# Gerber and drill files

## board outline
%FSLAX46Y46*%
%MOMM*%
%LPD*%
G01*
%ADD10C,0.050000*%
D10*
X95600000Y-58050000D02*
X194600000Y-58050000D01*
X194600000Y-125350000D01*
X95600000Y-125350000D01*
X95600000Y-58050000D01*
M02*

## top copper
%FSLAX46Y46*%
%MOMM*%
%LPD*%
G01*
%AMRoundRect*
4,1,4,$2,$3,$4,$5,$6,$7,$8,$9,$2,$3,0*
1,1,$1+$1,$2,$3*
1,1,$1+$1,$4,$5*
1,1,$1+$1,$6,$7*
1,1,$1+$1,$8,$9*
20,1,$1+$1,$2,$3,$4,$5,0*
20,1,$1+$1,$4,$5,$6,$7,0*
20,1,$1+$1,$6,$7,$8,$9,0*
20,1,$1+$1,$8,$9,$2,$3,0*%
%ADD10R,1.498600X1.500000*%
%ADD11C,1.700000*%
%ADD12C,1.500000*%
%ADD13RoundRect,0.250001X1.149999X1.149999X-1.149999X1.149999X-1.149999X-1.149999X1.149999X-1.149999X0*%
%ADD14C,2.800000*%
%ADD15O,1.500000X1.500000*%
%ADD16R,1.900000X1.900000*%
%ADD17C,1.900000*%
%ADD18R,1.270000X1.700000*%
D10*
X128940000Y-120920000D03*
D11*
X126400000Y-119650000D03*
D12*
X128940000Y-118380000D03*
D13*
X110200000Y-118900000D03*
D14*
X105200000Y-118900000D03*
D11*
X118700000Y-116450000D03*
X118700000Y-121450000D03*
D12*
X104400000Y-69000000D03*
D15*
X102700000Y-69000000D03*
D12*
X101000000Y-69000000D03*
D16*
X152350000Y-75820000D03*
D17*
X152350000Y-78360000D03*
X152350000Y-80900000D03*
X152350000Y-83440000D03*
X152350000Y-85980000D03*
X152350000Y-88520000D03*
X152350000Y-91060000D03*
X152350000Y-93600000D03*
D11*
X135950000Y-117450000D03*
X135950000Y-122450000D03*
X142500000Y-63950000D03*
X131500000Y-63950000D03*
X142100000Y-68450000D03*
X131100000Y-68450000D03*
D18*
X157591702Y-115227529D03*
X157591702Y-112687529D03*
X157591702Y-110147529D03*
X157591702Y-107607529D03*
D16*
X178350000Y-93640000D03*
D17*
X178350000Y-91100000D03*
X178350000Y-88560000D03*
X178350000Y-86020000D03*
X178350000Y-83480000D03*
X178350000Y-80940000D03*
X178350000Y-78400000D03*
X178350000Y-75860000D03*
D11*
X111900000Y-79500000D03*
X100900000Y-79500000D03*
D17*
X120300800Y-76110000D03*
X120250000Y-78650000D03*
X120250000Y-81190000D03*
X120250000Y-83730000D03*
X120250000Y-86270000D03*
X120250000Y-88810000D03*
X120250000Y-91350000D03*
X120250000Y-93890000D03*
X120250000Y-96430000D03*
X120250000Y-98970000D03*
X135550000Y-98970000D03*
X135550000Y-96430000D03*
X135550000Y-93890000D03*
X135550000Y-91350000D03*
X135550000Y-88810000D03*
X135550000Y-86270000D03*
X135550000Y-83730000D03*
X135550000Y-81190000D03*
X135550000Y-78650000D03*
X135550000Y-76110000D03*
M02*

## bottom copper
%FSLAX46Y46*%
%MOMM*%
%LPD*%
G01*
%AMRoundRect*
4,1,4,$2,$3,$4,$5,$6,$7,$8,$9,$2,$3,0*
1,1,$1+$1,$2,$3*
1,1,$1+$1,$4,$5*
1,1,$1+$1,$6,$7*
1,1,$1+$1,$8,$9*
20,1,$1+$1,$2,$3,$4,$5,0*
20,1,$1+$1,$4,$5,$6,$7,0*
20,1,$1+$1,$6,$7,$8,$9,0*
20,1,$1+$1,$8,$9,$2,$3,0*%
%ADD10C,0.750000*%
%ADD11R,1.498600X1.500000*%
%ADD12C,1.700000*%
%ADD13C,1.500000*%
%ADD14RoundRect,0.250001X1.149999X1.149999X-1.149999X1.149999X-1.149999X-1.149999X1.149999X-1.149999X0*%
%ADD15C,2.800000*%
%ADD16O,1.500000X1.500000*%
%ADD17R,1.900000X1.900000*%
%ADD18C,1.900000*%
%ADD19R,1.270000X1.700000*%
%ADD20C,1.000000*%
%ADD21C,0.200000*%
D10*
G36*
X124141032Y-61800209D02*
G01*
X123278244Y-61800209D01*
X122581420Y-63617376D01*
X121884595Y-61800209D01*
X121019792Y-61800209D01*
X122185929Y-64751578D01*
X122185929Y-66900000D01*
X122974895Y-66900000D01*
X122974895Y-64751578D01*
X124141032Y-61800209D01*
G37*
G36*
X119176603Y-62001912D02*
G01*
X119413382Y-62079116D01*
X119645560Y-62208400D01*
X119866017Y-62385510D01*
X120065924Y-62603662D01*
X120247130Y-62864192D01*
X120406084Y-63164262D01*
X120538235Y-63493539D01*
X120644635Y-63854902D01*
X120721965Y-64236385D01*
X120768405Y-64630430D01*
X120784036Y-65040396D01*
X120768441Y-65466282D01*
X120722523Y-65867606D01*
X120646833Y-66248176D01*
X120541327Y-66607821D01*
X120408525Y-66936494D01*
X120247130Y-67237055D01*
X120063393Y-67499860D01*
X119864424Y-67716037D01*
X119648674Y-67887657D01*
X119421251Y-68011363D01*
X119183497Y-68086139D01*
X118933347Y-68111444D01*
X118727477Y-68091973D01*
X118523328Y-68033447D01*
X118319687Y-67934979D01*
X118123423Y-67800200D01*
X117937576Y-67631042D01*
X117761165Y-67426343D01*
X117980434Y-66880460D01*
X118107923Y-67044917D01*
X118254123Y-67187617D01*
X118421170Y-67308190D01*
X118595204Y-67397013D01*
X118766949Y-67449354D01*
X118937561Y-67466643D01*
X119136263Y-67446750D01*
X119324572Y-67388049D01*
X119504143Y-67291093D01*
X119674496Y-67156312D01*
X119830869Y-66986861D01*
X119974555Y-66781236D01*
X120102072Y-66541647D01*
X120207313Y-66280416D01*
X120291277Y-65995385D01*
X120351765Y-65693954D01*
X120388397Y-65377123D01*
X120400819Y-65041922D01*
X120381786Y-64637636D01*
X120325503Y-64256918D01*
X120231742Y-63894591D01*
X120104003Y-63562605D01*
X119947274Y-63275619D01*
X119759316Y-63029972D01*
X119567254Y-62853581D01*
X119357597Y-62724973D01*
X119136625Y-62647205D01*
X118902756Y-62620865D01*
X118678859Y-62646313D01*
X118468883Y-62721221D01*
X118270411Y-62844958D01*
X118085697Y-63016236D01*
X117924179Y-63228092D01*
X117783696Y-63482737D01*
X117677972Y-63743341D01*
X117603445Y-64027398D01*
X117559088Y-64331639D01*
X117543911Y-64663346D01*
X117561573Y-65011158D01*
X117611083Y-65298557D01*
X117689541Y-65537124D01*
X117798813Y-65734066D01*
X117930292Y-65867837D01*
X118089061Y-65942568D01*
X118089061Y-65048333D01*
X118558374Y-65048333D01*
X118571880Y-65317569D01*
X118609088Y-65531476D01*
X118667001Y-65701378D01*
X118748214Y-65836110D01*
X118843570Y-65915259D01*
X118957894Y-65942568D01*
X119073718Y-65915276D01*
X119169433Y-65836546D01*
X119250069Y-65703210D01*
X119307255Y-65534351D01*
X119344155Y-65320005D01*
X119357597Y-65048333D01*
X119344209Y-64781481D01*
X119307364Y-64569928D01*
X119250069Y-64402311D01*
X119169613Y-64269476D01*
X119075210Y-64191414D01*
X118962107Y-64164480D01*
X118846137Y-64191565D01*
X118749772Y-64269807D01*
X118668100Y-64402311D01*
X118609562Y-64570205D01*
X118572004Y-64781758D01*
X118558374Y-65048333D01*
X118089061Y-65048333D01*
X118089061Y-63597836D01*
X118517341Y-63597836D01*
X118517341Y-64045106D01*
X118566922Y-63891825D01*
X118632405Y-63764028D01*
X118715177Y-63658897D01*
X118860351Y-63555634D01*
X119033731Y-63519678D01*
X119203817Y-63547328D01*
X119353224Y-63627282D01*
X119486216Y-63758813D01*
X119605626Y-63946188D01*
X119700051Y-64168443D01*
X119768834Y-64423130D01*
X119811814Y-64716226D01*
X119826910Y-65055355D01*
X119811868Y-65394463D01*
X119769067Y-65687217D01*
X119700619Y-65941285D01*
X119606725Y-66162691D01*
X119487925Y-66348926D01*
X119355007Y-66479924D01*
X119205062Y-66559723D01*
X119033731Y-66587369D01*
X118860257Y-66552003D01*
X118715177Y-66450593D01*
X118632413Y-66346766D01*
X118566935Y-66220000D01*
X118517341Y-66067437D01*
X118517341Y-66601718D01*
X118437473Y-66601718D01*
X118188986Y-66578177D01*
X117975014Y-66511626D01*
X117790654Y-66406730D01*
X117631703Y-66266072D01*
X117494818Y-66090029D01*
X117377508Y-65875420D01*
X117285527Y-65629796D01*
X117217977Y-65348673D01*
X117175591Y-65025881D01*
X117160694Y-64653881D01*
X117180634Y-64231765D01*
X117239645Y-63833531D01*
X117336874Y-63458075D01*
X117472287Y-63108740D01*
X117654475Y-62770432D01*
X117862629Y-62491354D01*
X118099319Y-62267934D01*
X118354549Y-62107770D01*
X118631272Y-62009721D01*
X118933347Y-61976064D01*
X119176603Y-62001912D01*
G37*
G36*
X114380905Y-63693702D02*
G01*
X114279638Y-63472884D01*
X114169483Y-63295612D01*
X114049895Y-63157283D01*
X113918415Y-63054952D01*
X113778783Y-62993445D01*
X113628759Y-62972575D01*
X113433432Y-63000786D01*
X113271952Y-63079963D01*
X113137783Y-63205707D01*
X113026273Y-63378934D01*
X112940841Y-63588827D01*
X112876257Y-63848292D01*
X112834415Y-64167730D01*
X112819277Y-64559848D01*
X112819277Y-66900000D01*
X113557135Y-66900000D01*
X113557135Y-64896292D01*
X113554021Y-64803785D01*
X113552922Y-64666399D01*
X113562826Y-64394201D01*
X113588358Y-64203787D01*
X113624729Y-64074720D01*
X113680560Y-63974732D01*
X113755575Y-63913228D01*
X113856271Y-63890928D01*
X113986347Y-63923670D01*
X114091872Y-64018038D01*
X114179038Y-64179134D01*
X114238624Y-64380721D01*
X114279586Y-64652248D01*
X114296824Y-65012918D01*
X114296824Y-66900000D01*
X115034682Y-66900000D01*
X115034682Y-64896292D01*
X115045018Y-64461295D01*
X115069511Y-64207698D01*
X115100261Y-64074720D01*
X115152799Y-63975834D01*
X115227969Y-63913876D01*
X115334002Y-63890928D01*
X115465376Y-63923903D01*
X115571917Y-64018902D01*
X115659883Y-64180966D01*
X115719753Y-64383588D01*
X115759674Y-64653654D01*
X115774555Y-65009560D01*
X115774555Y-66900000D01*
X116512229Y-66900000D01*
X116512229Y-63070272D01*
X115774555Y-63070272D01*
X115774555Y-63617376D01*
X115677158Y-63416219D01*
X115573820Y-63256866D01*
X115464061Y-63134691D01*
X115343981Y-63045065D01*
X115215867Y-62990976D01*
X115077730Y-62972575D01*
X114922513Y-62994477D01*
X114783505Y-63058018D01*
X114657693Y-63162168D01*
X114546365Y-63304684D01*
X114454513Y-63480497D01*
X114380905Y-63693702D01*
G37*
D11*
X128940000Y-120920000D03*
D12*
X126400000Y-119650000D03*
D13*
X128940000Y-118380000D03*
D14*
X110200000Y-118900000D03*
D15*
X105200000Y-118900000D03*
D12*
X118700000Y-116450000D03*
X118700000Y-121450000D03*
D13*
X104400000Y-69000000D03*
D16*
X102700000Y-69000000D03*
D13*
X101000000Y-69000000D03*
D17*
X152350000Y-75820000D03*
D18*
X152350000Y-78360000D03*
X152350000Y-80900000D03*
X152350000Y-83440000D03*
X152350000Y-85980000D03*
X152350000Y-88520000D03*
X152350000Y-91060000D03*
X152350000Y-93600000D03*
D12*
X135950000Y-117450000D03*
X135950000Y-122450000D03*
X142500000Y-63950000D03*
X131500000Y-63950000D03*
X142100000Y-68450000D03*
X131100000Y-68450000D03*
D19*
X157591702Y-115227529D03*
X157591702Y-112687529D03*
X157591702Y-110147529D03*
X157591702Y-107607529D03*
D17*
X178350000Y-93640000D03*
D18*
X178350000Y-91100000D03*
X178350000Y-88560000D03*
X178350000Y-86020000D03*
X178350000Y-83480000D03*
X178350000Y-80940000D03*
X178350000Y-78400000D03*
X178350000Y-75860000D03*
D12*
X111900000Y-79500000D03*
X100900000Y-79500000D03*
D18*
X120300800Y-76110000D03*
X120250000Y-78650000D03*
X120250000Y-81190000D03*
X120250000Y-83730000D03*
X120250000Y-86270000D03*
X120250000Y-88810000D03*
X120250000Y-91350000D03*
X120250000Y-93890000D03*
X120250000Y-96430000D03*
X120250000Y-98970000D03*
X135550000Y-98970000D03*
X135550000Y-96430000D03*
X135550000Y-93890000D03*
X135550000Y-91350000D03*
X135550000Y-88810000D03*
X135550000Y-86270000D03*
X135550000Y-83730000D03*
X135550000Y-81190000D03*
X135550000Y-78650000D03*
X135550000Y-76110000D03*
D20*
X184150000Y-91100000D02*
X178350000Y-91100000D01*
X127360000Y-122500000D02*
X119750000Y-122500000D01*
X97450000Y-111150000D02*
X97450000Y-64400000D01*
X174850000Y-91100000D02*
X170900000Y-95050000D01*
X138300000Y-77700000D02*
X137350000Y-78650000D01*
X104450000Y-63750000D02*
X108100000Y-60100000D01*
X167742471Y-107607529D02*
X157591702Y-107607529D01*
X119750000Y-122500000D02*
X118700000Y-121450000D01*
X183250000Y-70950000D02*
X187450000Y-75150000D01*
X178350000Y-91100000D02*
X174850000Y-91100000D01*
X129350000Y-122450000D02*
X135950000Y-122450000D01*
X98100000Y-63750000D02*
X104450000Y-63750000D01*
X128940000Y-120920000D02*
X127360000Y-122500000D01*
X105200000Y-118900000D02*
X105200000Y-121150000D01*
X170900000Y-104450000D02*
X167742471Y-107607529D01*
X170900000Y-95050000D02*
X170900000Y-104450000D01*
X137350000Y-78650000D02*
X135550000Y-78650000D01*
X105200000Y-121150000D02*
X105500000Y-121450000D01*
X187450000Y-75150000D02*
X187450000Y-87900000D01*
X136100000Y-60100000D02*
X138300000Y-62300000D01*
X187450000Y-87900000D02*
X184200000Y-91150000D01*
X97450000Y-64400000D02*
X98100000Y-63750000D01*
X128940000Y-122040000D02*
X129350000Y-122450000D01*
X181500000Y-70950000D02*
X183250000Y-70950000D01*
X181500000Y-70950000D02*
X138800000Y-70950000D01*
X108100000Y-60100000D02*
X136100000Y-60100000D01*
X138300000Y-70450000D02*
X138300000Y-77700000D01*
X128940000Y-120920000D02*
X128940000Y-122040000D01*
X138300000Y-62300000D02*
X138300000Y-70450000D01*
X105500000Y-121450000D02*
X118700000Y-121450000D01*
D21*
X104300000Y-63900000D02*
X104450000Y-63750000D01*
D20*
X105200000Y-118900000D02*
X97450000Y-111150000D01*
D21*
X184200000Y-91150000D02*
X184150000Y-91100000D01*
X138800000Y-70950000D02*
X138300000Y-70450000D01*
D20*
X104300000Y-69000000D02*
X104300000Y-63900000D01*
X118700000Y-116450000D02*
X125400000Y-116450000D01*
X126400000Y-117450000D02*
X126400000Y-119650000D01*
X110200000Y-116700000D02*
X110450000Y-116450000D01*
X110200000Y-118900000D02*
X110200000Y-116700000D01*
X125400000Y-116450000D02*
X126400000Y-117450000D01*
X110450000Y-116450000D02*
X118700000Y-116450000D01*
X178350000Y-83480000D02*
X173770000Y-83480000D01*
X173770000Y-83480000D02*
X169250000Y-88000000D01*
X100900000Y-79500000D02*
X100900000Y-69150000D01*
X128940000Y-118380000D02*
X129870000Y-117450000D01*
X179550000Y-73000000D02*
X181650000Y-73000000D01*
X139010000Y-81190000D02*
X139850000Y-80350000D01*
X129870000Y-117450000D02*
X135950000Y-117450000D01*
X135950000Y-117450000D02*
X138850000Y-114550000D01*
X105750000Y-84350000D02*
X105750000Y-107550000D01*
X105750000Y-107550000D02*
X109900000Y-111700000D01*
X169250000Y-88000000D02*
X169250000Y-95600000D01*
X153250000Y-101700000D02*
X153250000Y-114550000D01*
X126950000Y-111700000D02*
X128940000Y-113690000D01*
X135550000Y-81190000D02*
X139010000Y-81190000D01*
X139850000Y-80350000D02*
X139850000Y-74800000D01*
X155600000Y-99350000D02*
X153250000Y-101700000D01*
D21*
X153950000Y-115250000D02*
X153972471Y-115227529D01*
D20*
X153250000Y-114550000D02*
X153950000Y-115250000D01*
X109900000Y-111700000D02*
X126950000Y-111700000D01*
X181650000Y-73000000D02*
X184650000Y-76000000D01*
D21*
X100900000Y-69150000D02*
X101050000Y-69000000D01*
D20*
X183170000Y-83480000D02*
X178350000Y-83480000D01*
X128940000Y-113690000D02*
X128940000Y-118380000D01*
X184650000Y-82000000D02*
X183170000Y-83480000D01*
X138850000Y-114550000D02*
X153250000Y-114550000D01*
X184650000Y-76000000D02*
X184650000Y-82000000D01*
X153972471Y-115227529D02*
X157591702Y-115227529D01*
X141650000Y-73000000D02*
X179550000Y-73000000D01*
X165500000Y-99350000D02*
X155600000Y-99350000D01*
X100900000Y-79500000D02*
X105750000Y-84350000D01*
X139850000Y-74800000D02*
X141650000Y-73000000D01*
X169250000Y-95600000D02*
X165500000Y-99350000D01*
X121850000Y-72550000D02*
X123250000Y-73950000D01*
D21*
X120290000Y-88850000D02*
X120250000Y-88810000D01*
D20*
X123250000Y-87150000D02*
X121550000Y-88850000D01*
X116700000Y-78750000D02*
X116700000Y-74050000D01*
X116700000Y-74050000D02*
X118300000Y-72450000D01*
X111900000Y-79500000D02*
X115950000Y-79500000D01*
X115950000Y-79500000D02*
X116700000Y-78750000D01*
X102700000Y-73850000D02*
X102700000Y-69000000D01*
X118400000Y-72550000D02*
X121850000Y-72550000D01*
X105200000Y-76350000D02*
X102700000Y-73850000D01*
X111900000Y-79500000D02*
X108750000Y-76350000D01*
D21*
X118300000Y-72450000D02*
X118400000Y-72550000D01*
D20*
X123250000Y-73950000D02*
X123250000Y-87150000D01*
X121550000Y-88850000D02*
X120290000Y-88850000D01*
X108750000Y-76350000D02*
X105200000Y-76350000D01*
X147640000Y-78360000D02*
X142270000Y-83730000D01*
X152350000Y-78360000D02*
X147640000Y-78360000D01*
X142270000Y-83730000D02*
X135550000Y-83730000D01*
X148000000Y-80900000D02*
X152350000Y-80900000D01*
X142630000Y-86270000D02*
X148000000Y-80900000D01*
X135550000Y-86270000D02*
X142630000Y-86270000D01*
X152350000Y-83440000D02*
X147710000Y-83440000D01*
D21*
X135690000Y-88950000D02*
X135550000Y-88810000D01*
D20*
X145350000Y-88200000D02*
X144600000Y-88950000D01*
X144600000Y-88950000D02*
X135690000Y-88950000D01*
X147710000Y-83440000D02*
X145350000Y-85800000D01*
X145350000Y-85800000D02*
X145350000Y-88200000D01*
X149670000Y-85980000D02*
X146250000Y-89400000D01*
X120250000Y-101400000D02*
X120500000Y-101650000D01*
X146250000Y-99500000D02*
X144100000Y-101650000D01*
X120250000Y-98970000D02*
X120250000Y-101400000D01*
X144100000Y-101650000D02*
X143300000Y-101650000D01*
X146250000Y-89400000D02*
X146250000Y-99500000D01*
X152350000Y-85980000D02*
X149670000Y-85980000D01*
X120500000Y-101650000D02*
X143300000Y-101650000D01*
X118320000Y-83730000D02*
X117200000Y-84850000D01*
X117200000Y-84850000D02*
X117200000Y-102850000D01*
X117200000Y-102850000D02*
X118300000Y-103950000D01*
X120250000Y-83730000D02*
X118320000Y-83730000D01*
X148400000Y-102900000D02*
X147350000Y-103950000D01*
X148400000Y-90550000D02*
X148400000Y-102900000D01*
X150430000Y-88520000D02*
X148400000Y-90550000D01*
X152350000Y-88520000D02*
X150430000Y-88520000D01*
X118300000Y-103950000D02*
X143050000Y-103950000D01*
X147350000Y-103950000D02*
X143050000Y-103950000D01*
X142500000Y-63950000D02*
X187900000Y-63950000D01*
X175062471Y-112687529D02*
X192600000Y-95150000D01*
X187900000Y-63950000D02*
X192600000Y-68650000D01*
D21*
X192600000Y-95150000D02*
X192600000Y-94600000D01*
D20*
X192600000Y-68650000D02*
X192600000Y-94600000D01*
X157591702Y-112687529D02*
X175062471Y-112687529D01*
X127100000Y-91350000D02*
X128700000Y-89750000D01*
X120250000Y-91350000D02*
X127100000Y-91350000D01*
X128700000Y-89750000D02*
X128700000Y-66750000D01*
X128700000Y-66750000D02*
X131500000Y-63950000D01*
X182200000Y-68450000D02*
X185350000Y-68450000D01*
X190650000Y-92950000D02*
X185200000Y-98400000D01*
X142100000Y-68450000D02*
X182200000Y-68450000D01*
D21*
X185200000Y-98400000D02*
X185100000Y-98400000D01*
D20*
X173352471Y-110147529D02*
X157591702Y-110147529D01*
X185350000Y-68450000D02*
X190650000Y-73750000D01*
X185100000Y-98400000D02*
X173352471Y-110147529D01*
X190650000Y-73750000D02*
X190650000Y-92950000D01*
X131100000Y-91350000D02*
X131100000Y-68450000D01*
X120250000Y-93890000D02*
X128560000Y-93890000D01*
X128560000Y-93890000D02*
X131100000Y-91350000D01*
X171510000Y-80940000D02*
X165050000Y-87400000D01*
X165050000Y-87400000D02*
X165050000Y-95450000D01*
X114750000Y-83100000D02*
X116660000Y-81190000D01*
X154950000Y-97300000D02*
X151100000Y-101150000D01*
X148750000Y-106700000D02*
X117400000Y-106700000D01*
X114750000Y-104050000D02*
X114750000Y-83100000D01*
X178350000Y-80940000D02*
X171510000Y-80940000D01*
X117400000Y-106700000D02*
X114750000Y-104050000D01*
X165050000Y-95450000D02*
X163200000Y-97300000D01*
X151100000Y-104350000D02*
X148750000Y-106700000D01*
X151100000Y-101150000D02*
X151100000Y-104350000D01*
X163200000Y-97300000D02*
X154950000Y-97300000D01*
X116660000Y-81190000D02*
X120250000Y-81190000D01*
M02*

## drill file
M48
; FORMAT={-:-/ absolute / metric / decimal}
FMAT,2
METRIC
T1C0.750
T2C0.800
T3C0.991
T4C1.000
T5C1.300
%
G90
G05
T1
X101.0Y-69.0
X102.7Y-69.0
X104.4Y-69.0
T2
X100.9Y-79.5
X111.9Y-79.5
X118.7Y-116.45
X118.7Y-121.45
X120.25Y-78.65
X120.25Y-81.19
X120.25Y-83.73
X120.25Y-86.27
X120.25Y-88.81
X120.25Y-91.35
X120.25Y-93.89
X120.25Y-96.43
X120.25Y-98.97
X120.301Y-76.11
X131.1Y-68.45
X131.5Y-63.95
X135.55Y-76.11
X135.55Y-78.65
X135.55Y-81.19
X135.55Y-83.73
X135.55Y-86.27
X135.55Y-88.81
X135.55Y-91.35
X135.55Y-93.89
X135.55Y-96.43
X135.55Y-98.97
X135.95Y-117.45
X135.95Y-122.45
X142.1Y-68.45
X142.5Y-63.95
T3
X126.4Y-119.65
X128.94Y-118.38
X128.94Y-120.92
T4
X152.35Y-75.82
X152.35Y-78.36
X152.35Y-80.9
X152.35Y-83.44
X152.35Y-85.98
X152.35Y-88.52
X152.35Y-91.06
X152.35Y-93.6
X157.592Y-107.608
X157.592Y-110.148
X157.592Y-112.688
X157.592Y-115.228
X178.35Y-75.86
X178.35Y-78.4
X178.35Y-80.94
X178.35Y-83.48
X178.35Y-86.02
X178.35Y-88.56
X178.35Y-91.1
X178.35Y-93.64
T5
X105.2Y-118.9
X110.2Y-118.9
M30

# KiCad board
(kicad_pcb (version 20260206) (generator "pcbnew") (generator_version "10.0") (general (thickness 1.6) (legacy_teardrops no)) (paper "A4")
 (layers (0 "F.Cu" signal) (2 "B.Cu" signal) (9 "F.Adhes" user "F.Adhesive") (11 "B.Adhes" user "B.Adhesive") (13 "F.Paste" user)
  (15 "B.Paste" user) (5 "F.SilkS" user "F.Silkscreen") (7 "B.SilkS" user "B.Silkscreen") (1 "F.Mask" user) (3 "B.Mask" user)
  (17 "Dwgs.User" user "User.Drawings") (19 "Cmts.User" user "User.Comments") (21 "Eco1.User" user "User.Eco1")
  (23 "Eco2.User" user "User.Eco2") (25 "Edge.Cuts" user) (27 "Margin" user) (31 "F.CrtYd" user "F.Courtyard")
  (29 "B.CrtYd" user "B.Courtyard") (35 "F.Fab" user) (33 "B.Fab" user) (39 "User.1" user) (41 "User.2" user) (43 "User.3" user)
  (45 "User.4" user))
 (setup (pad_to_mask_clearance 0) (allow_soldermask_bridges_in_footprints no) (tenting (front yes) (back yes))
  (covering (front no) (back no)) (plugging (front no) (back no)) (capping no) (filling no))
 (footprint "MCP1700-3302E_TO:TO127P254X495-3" (layer "F.Cu") (at 126.4 118.38 90)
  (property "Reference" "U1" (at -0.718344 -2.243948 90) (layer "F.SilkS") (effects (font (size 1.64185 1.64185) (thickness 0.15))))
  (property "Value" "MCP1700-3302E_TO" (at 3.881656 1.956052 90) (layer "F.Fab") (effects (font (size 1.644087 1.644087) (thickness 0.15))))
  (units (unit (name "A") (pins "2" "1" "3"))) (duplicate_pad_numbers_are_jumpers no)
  (pad "1" thru_hole rect (at -2.54 2.54 90) (size 1.5 1.4986) (drill 0.9906) (layers "*.Cu" "*.Mask") (remove_unused_layers no) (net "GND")
   (solder_mask_margin 0.102))
  (pad "2" thru_hole circle (at -1.27 0 90) (size 1.7 1.7) (drill 0.9906) (layers "*.Cu" "*.Mask") (remove_unused_layers no) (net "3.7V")
   (solder_mask_margin 0.102))
  (pad "3" thru_hole circle (at 0 2.54 90) (size 1.5 1.5) (drill 0.9906) (layers "*.Cu" "*.Mask") (remove_unused_layers no) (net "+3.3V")
   (solder_mask_margin 0.102)))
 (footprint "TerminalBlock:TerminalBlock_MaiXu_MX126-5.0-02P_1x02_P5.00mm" (layer "F.Cu") (at 110.2 118.9 180)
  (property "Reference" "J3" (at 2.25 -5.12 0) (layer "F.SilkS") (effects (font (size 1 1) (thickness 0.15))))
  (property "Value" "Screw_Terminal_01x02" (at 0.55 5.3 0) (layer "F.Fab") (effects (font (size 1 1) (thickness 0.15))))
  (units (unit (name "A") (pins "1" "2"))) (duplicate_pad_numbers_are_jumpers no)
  (pad "1" thru_hole roundrect (at 0 0 180) (size 2.8 2.8) (drill 1.3) (layers "*.Cu" "*.Mask") (remove_unused_layers no)
   (roundrect_rratio 0.089286) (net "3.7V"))
  (pad "2" thru_hole circle (at 5 0 180) (size 2.8 2.8) (drill 1.3) (layers "*.Cu" "*.Mask") (remove_unused_layers no) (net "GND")))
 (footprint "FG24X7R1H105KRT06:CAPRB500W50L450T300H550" (layer "F.Cu") (at 118.7 118.95 -90)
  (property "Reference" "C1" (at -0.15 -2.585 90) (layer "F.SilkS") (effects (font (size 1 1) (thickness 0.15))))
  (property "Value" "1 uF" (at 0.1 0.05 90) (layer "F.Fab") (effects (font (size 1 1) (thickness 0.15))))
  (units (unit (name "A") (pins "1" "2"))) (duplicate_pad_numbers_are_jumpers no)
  (pad "1" thru_hole circle (at -2.5 0 270) (size 1.7 1.7) (drill 0.8) (layers "*.Cu" "*.Mask") (remove_unused_layers no) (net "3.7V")
   (solder_mask_margin 0.102))
  (pad "2" thru_hole circle (at 2.5 0 270) (size 1.7 1.7) (drill 0.8) (layers "*.Cu" "*.Mask") (remove_unused_layers no) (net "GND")
   (solder_mask_margin 0.102)))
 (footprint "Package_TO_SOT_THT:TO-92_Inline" (layer "F.Cu") (at 103.97 69 180)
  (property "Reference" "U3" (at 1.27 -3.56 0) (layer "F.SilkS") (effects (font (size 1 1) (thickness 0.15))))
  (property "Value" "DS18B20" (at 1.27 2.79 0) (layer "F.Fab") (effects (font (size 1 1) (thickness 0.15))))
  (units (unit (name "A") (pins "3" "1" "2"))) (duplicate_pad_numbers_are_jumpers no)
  (pad "1" thru_hole circle (at -0.43 0 180) (size 1.5 1.5) (drill 0.75) (layers "*.Cu" "*.Mask") (remove_unused_layers no) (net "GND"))
  (pad "2" thru_hole oval (at 1.27 0 180) (size 1.5 1.5) (drill 0.75) (layers "*.Cu" "*.Mask") (remove_unused_layers no) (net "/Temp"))
  (pad "3" thru_hole circle (at 2.97 0 180) (size 1.5 1.5) (drill 0.75) (layers "*.Cu" "*.Mask") (remove_unused_layers no) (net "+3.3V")))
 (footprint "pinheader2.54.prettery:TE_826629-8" (layer "F.Cu") (at 152.35 75.82 -90)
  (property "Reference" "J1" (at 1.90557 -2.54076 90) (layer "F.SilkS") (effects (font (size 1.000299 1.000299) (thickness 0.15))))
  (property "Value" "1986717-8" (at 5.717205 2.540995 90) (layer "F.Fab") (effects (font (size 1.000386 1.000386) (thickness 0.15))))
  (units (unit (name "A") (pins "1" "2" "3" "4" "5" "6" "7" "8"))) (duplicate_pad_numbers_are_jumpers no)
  (pad "1" thru_hole rect (at 0 0 270) (size 1.9 1.9) (drill 1) (layers "*.Cu" "*.Mask") (remove_unused_layers no)
   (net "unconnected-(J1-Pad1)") (solder_mask_margin 0.102))
  (pad "2" thru_hole circle (at 2.54 0 270) (size 1.9 1.9) (drill 1) (layers "*.Cu" "*.Mask") (remove_unused_layers no) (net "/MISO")
   (solder_mask_margin 0.102))
  (pad "3" thru_hole circle (at 5.08 0 270) (size 1.9 1.9) (drill 1) (layers "*.Cu" "*.Mask") (remove_unused_layers no) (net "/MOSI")
   (solder_mask_margin 0.102))
  (pad "4" thru_hole circle (at 7.62 0 270) (size 1.9 1.9) (drill 1) (layers "*.Cu" "*.Mask") (remove_unused_layers no) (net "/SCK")
   (solder_mask_margin 0.102))
  (pad "5" thru_hole circle (at 10.16 0 270) (size 1.9 1.9) (drill 1) (layers "*.Cu" "*.Mask") (remove_unused_layers no) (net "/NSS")
   (solder_mask_margin 0.102))
  (pad "6" thru_hole circle (at 12.7 0 270) (size 1.9 1.9) (drill 1) (layers "*.Cu" "*.Mask") (remove_unused_layers no) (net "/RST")
   (solder_mask_margin 0.102))
  (pad "7" thru_hole circle (at 15.24 0 270) (size 1.9 1.9) (drill 1) (layers "*.Cu" "*.Mask") (remove_unused_layers no)
   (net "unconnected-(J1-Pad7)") (solder_mask_margin 0.102))
  (pad "8" thru_hole circle (at 17.78 0 270) (size 1.9 1.9) (drill 1) (layers "*.Cu" "*.Mask") (remove_unused_layers no)
   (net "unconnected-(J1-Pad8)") (solder_mask_margin 0.102)))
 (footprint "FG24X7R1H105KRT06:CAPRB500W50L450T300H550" (layer "F.Cu") (at 135.95 119.95 -90)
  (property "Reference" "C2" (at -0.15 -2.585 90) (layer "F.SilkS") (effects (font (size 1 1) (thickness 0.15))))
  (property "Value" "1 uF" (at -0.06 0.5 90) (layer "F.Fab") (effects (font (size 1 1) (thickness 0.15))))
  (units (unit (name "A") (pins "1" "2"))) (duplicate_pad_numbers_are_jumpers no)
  (pad "1" thru_hole circle (at -2.5 0 270) (size 1.7 1.7) (drill 0.8) (layers "*.Cu" "*.Mask") (remove_unused_layers no) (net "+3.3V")
   (solder_mask_margin 0.102))
  (pad "2" thru_hole circle (at 2.5 0 270) (size 1.7 1.7) (drill 0.8) (layers "*.Cu" "*.Mask") (remove_unused_layers no) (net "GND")
   (solder_mask_margin 0.102)))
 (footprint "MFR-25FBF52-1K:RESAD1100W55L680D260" (layer "F.Cu") (at 137 63.95 180)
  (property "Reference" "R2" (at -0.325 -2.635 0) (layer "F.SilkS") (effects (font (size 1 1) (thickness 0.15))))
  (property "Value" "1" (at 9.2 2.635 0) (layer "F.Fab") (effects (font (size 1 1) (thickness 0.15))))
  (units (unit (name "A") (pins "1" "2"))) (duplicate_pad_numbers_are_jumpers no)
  (pad "1" thru_hole circle (at -5.5 0 180) (size 1.7 1.7) (drill 0.8) (layers "*.Cu" "*.Mask") (remove_unused_layers no) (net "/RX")
   (solder_mask_margin 0.102))
  (pad "2" thru_hole circle (at 5.5 0 180) (size 1.7 1.7) (drill 0.8) (layers "*.Cu" "*.Mask") (remove_unused_layers no)
   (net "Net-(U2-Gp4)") (solder_mask_margin 0.102)))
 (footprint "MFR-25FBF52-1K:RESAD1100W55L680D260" (layer "F.Cu") (at 136.6 68.45 180)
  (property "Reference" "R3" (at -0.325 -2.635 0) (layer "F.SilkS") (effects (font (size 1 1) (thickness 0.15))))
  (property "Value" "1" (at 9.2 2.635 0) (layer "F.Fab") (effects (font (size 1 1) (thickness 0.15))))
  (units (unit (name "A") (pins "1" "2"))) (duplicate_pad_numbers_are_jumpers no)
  (pad "1" thru_hole circle (at -5.5 0 180) (size 1.7 1.7) (drill 0.8) (layers "*.Cu" "*.Mask") (remove_unused_layers no) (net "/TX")
   (solder_mask_margin 0.102))
  (pad "2" thru_hole circle (at 5.5 0 180) (size 1.7 1.7) (drill 0.8) (layers "*.Cu" "*.Mask") (remove_unused_layers no)
   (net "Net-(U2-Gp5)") (solder_mask_margin 0.102)))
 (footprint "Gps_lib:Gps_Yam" (layer "F.Cu") (at 156.091702 123.863529 90)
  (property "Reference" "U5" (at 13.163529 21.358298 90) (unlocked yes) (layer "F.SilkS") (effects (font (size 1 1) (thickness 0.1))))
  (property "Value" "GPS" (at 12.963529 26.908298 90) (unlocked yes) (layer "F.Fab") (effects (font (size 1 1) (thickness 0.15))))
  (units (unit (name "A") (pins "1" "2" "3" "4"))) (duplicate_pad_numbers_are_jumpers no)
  (pad "1" thru_hole rect (at 8.636 1.5 90) (size 1.7 1.27) (drill 1) (layers "*.Cu" "*.Mask") (remove_unused_layers no) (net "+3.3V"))
  (pad "2" thru_hole rect (at 11.176 1.5 90) (size 1.7 1.27) (drill 1) (layers "*.Cu" "*.Mask") (remove_unused_layers no) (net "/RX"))
  (pad "3" thru_hole rect (at 13.716 1.5 90) (size 1.7 1.27) (drill 1) (layers "*.Cu" "*.Mask") (remove_unused_layers no) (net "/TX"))
  (pad "4" thru_hole rect (at 16.256 1.5 90) (size 1.7 1.27) (drill 1) (layers "*.Cu" "*.Mask") (remove_unused_layers no) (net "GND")))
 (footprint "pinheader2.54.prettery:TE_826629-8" (layer "F.Cu") (at 178.35 93.64 90)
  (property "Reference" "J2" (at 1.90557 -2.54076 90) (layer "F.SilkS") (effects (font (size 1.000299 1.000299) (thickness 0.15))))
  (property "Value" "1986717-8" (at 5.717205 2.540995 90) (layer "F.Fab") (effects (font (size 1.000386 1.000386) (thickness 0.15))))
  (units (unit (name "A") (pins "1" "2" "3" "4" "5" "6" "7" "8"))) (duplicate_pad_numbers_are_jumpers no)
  (pad "1" thru_hole rect (at 0 0 90) (size 1.9 1.9) (drill 1) (layers "*.Cu" "*.Mask") (remove_unused_layers no)
   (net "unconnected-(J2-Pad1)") (solder_mask_margin 0.102))
  (pad "2" thru_hole circle (at 2.54 0 90) (size 1.9 1.9) (drill 1) (layers "*.Cu" "*.Mask") (remove_unused_layers no) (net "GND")
   (solder_mask_margin 0.102))
  (pad "3" thru_hole circle (at 5.08 0 90) (size 1.9 1.9) (drill 1) (layers "*.Cu" "*.Mask") (remove_unused_layers no)
   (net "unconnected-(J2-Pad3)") (solder_mask_margin 0.102))
  (pad "4" thru_hole circle (at 7.62 0 90) (size 1.9 1.9) (drill 1) (layers "*.Cu" "*.Mask") (remove_unused_layers no)
   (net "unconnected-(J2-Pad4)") (solder_mask_margin 0.102))
  (pad "5" thru_hole circle (at 10.16 0 90) (size 1.9 1.9) (drill 1) (layers "*.Cu" "*.Mask") (remove_unused_layers no) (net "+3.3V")
   (solder_mask_margin 0.102))
  (pad "6" thru_hole circle (at 12.7 0 90) (size 1.9 1.9) (drill 1) (layers "*.Cu" "*.Mask") (remove_unused_layers no) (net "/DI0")
   (solder_mask_margin 0.102))
  (pad "7" thru_hole circle (at 15.24 0 90) (size 1.9 1.9) (drill 1) (layers "*.Cu" "*.Mask") (remove_unused_layers no)
   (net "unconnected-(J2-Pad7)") (solder_mask_margin 0.102))
  (pad "8" thru_hole circle (at 17.78 0 90) (size 1.9 1.9) (drill 1) (layers "*.Cu" "*.Mask") (remove_unused_layers no)
   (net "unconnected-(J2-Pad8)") (solder_mask_margin 0.102)))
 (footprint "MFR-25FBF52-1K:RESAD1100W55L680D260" (layer "F.Cu") (at 106.4 79.5 180)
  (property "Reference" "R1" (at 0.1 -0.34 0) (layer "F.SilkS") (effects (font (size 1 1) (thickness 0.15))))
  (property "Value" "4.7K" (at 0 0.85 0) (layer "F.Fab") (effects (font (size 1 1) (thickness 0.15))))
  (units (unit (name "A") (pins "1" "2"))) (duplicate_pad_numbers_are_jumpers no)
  (pad "1" thru_hole circle (at -5.5 0 180) (size 1.7 1.7) (drill 0.8) (layers "*.Cu" "*.Mask") (remove_unused_layers no) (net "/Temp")
   (solder_mask_margin 0.102))
  (pad "2" thru_hole circle (at 5.5 0 180) (size 1.7 1.7) (drill 0.8) (layers "*.Cu" "*.Mask") (remove_unused_layers no) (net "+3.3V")
   (solder_mask_margin 0.102)))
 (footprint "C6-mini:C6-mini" (layer "F.Cu") (at 120.25 72.935)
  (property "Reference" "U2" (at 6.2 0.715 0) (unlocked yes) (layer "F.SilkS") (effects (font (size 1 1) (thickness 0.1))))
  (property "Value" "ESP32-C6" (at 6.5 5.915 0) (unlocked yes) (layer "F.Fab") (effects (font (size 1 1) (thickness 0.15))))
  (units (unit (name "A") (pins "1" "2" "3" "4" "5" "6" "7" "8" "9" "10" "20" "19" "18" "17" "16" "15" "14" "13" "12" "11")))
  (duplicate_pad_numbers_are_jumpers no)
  (pad "1" thru_hole circle (at 0.0508 3.175) (size 1.9 1.9) (drill 0.8) (layers "*.Cu" "*.Mask") (remove_unused_layers no)
   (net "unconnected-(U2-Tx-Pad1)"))
  (pad "2" thru_hole circle (at 0 5.715) (size 1.9 1.9) (drill 0.8) (layers "*.Cu" "*.Mask") (remove_unused_layers no)
   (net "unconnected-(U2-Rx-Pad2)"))
  (pad "3" thru_hole circle (at 0 8.255) (size 1.9 1.9) (drill 0.8) (layers "*.Cu" "*.Mask") (remove_unused_layers no) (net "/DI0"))
  (pad "4" thru_hole circle (at 0 10.795) (size 1.9 1.9) (drill 0.8) (layers "*.Cu" "*.Mask") (remove_unused_layers no) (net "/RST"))
  (pad "5" thru_hole circle (at 0 13.335) (size 1.9 1.9) (drill 0.8) (layers "*.Cu" "*.Mask") (remove_unused_layers no)
   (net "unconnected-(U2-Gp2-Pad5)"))
  (pad "6" thru_hole circle (at 0 15.875) (size 1.9 1.9) (drill 0.8) (layers "*.Cu" "*.Mask") (remove_unused_layers no) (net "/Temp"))
  (pad "7" thru_hole circle (at 0 18.415) (size 1.9 1.9) (drill 0.8) (layers "*.Cu" "*.Mask") (remove_unused_layers no) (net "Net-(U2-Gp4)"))
  (pad "8" thru_hole circle (at 0 20.955) (size 1.9 1.9) (drill 0.8) (layers "*.Cu" "*.Mask") (remove_unused_layers no) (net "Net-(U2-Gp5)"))
  (pad "9" thru_hole circle (at 0 23.495) (size 1.9 1.9) (drill 0.8) (layers "*.Cu" "*.Mask") (remove_unused_layers no)
   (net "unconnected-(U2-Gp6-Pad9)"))
  (pad "10" thru_hole circle (at 0 26.035) (size 1.9 1.9) (drill 0.8) (layers "*.Cu" "*.Mask") (remove_unused_layers no) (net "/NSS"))
  (pad "11" thru_hole circle (at 15.3 26.035) (size 1.9 1.9) (drill 0.8) (layers "*.Cu" "*.Mask") (remove_unused_layers no)
   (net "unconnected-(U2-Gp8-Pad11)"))
  (pad "12" thru_hole circle (at 15.3 23.495) (size 1.9 1.9) (drill 0.8) (layers "*.Cu" "*.Mask") (remove_unused_layers no)
   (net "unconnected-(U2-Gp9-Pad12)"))
  (pad "13" thru_hole circle (at 15.3 20.955) (size 1.9 1.9) (drill 0.8) (layers "*.Cu" "*.Mask") (remove_unused_layers no)
   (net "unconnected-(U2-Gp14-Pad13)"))
  (pad "14" thru_hole circle (at 15.3 18.415) (size 1.9 1.9) (drill 0.8) (layers "*.Cu" "*.Mask") (remove_unused_layers no)
   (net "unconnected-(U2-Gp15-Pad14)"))
  (pad "15" thru_hole circle (at 15.3 15.875) (size 1.9 1.9) (drill 0.8) (layers "*.Cu" "*.Mask") (remove_unused_layers no) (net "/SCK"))
  (pad "16" thru_hole circle (at 15.3 13.335) (size 1.9 1.9) (drill 0.8) (layers "*.Cu" "*.Mask") (remove_unused_layers no) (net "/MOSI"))
  (pad "17" thru_hole circle (at 15.3 10.795) (size 1.9 1.9) (drill 0.8) (layers "*.Cu" "*.Mask") (remove_unused_layers no) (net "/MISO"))
  (pad "18" thru_hole circle (at 15.3 8.255) (size 1.9 1.9) (drill 0.8) (layers "*.Cu" "*.Mask") (remove_unused_layers no) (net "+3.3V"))
  (pad "19" thru_hole circle (at 15.3 5.715) (size 1.9 1.9) (drill 0.8) (layers "*.Cu" "*.Mask") (remove_unused_layers no) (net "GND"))
  (pad "20" thru_hole circle (at 15.3 3.175) (size 1.9 1.9) (drill 0.8) (layers "*.Cu" "*.Mask") (remove_unused_layers no)
   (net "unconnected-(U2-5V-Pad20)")))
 (gr_rect (start 95.6 58.05) (end 194.6 125.35) (stroke (width 0.05) (type default)) (fill no) (layer "Edge.Cuts"))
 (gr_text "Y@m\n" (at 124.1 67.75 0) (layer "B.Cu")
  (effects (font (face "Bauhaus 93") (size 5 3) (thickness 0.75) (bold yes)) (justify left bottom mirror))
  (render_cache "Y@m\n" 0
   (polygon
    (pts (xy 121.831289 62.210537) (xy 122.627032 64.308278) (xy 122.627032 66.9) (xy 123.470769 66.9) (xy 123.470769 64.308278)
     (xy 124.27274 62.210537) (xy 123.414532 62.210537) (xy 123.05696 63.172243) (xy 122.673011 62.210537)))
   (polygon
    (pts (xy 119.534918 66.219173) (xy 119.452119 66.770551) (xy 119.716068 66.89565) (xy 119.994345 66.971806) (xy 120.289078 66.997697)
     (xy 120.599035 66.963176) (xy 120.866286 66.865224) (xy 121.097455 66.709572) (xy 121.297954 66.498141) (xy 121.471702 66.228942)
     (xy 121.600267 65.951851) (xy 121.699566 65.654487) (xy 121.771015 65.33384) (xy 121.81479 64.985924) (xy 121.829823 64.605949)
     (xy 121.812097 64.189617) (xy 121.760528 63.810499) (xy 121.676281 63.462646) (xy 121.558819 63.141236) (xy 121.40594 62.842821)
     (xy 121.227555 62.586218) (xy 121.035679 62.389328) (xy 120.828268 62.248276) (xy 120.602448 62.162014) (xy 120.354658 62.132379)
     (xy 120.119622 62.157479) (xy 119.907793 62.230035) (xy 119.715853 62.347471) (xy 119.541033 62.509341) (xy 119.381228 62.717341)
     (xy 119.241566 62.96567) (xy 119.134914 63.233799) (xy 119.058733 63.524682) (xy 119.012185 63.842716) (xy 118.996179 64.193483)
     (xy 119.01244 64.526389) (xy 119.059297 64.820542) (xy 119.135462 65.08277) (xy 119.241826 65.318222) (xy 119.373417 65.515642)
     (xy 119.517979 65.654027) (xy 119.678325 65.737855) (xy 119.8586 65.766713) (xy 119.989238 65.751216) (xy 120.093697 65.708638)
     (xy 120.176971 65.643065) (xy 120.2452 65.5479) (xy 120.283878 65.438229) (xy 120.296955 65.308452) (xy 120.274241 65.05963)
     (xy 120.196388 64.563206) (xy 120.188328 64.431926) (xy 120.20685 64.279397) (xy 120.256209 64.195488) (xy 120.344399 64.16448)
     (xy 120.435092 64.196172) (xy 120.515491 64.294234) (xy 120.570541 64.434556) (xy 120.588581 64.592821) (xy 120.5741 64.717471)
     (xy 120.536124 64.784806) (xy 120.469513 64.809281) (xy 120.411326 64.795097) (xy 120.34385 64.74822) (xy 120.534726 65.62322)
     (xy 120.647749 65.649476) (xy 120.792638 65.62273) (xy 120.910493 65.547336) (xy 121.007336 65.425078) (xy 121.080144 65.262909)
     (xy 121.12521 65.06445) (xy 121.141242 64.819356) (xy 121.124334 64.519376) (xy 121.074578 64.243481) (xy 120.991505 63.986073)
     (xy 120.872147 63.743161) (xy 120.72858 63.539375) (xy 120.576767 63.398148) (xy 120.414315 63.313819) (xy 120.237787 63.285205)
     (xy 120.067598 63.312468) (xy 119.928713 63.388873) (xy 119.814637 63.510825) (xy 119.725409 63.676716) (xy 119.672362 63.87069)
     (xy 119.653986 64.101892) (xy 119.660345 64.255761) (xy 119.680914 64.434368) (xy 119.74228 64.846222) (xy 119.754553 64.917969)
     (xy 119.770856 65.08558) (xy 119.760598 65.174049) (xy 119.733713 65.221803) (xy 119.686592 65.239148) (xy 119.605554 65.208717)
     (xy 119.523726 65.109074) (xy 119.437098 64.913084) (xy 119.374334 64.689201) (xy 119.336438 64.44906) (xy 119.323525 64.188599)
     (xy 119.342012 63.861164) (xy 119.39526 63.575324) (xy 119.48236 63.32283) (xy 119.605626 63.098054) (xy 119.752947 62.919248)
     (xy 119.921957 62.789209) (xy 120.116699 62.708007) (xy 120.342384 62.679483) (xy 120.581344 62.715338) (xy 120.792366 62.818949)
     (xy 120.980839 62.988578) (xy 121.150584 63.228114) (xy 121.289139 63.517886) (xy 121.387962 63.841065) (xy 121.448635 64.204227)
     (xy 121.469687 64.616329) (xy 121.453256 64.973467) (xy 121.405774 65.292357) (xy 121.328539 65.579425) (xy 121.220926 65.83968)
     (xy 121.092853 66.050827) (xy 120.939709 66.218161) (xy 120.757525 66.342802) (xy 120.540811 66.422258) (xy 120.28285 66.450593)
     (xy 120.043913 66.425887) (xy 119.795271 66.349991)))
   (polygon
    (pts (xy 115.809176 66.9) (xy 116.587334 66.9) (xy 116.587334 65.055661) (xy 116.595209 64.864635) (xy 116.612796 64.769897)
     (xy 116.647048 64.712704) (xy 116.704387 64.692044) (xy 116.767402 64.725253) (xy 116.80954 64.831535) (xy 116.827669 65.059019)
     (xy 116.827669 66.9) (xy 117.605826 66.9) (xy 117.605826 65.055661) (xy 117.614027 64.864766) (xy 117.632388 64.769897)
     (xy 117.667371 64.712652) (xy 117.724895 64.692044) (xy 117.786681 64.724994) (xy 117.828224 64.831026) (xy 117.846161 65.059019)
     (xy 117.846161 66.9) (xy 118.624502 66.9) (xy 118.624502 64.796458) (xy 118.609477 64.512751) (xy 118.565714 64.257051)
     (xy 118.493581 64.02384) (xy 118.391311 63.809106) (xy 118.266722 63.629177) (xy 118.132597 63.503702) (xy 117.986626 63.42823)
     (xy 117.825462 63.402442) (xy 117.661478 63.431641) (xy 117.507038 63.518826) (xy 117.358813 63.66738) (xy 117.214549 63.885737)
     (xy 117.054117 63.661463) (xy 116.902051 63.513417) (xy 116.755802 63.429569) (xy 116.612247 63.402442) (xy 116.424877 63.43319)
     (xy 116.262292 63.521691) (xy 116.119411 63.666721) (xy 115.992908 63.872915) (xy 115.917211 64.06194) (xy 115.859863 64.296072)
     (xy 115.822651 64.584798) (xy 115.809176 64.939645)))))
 (segment (start 184.15 91.1) (end 178.35 91.1) (width 1) (layer "B.Cu") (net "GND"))
 (segment (start 127.36 122.5) (end 119.75 122.5) (width 1) (layer "B.Cu") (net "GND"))
 (segment (start 97.45 111.15) (end 97.45 64.4) (width 1) (layer "B.Cu") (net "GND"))
 (segment (start 174.85 91.1) (end 170.9 95.05) (width 1) (layer "B.Cu") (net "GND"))
 (segment (start 138.3 77.7) (end 137.35 78.65) (width 1) (layer "B.Cu") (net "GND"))
 (segment (start 104.45 63.75) (end 108.1 60.1) (width 1) (layer "B.Cu") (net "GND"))
 (segment (start 167.742471 107.607529) (end 157.591702 107.607529) (width 1) (layer "B.Cu") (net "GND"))
 (segment (start 119.75 122.5) (end 118.7 121.45) (width 1) (layer "B.Cu") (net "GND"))
 (segment (start 183.25 70.95) (end 187.45 75.15) (width 1) (layer "B.Cu") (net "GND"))
 (segment (start 178.35 91.1) (end 174.85 91.1) (width 1) (layer "B.Cu") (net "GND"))
 (segment (start 129.35 122.45) (end 135.95 122.45) (width 1) (layer "B.Cu") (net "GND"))
 (segment (start 98.1 63.75) (end 104.45 63.75) (width 1) (layer "B.Cu") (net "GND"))
 (segment (start 128.94 120.92) (end 127.36 122.5) (width 1) (layer "B.Cu") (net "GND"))
 (segment (start 105.2 118.9) (end 105.2 121.15) (width 1) (layer "B.Cu") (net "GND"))
 (segment (start 170.9 104.45) (end 167.742471 107.607529) (width 1) (layer "B.Cu") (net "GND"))
 (segment (start 170.9 95.05) (end 170.9 104.45) (width 1) (layer "B.Cu") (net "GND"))
 (segment (start 137.35 78.65) (end 135.55 78.65) (width 1) (layer "B.Cu") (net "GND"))
 (segment (start 105.2 121.15) (end 105.5 121.45) (width 1) (layer "B.Cu") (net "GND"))
 (segment (start 187.45 75.15) (end 187.45 87.9) (width 1) (layer "B.Cu") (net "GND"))
 (segment (start 136.1 60.1) (end 138.3 62.3) (width 1) (layer "B.Cu") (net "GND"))
 (segment (start 187.45 87.9) (end 184.2 91.15) (width 1) (layer "B.Cu") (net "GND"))
 (segment (start 97.45 64.4) (end 98.1 63.75) (width 1) (layer "B.Cu") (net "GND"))
 (segment (start 128.94 122.04) (end 129.35 122.45) (width 1) (layer "B.Cu") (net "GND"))
 (segment (start 181.5 70.95) (end 183.25 70.95) (width 1) (layer "B.Cu") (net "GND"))
 (segment (start 181.5 70.95) (end 138.8 70.95) (width 1) (layer "B.Cu") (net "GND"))
 (segment (start 108.1 60.1) (end 136.1 60.1) (width 1) (layer "B.Cu") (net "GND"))
 (segment (start 138.3 70.45) (end 138.3 77.7) (width 1) (layer "B.Cu") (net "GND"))
 (segment (start 128.94 120.92) (end 128.94 122.04) (width 1) (layer "B.Cu") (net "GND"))
 (segment (start 138.3 62.3) (end 138.3 70.45) (width 1) (layer "B.Cu") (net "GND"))
 (segment (start 105.5 121.45) (end 118.7 121.45) (width 1) (layer "B.Cu") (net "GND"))
 (segment (start 104.3 63.9) (end 104.45 63.75) (width 0.2) (layer "B.Cu") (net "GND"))
 (segment (start 105.2 118.9) (end 97.45 111.15) (width 1) (layer "B.Cu") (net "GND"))
 (segment (start 184.2 91.15) (end 184.15 91.1) (width 0.2) (layer "B.Cu") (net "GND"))
 (segment (start 138.8 70.95) (end 138.3 70.45) (width 0.2) (layer "B.Cu") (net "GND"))
 (segment (start 104.3 69) (end 104.3 63.9) (width 1) (layer "B.Cu") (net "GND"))
 (segment (start 118.7 116.45) (end 125.4 116.45) (width 1) (layer "B.Cu") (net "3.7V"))
 (segment (start 126.4 117.45) (end 126.4 119.65) (width 1) (layer "B.Cu") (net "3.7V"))
 (segment (start 110.2 116.7) (end 110.45 116.45) (width 1) (layer "B.Cu") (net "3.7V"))
 (segment (start 110.2 118.9) (end 110.2 116.7) (width 1) (layer "B.Cu") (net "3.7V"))
 (segment (start 125.4 116.45) (end 126.4 117.45) (width 1) (layer "B.Cu") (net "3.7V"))
 (segment (start 110.45 116.45) (end 118.7 116.45) (width 1) (layer "B.Cu") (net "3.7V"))
 (segment (start 178.35 83.48) (end 173.77 83.48) (width 1) (layer "B.Cu") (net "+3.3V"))
 (segment (start 173.77 83.48) (end 169.25 88) (width 1) (layer "B.Cu") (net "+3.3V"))
 (segment (start 100.9 79.5) (end 100.9 69.15) (width 1) (layer "B.Cu") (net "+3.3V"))
 (segment (start 128.94 118.38) (end 129.87 117.45) (width 1) (layer "B.Cu") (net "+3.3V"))
 (segment (start 179.55 73) (end 181.65 73) (width 1) (layer "B.Cu") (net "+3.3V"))
 (segment (start 139.01 81.19) (end 139.85 80.35) (width 1) (layer "B.Cu") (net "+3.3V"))
 (segment (start 129.87 117.45) (end 135.95 117.45) (width 1) (layer "B.Cu") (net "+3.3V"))
 (segment (start 135.95 117.45) (end 138.85 114.55) (width 1) (layer "B.Cu") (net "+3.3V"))
 (segment (start 105.75 84.35) (end 105.75 107.55) (width 1) (layer "B.Cu") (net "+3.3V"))
 (segment (start 105.75 107.55) (end 109.9 111.7) (width 1) (layer "B.Cu") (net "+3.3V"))
 (segment (start 169.25 88) (end 169.25 95.6) (width 1) (layer "B.Cu") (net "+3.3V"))
 (segment (start 153.25 101.7) (end 153.25 114.55) (width 1) (layer "B.Cu") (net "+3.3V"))
 (segment (start 126.95 111.7) (end 128.94 113.69) (width 1) (layer "B.Cu") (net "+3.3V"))
 (segment (start 135.55 81.19) (end 139.01 81.19) (width 1) (layer "B.Cu") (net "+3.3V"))
 (segment (start 139.85 80.35) (end 139.85 74.8) (width 1) (layer "B.Cu") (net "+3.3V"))
 (segment (start 155.6 99.35) (end 153.25 101.7) (width 1) (layer "B.Cu") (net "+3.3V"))
 (segment (start 153.95 115.25) (end 153.972471 115.227529) (width 0.2) (layer "B.Cu") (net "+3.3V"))
 (segment (start 153.25 114.55) (end 153.95 115.25) (width 1) (layer "B.Cu") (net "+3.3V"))
 (segment (start 109.9 111.7) (end 126.95 111.7) (width 1) (layer "B.Cu") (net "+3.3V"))
 (segment (start 181.65 73) (end 184.65 76) (width 1) (layer "B.Cu") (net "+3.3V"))
 (segment (start 100.9 69.15) (end 101.05 69) (width 0.2) (layer "B.Cu") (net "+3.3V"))
 (segment (start 183.17 83.48) (end 178.35 83.48) (width 1) (layer "B.Cu") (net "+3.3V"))
 (segment (start 128.94 113.69) (end 128.94 118.38) (width 1) (layer "B.Cu") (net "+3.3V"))
 (segment (start 184.65 82) (end 183.17 83.48) (width 1) (layer "B.Cu") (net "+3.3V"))
 (segment (start 138.85 114.55) (end 153.25 114.55) (width 1) (layer "B.Cu") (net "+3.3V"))
 (segment (start 184.65 76) (end 184.65 82) (width 1) (layer "B.Cu") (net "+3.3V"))
 (segment (start 153.972471 115.227529) (end 157.591702 115.227529) (width 1) (layer "B.Cu") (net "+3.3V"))
 (segment (start 141.65 73) (end 179.55 73) (width 1) (layer "B.Cu") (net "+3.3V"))
 (segment (start 165.5 99.35) (end 155.6 99.35) (width 1) (layer "B.Cu") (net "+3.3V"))
 (segment (start 100.9 79.5) (end 105.75 84.35) (width 1) (layer "B.Cu") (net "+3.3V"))
 (segment (start 139.85 74.8) (end 141.65 73) (width 1) (layer "B.Cu") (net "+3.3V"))
 (segment (start 169.25 95.6) (end 165.5 99.35) (width 1) (layer "B.Cu") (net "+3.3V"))
 (segment (start 121.85 72.55) (end 123.25 73.95) (width 1) (layer "B.Cu") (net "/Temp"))
 (segment (start 120.29 88.85) (end 120.25 88.81) (width 0.2) (layer "B.Cu") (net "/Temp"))
 (segment (start 123.25 87.15) (end 121.55 88.85) (width 1) (layer "B.Cu") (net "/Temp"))
 (segment (start 116.7 78.75) (end 116.7 74.05) (width 1) (layer "B.Cu") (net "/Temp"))
 (segment (start 116.7 74.05) (end 118.3 72.45) (width 1) (layer "B.Cu") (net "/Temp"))
 (segment (start 111.9 79.5) (end 115.95 79.5) (width 1) (layer "B.Cu") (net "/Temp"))
 (segment (start 115.95 79.5) (end 116.7 78.75) (width 1) (layer "B.Cu") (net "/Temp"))
 (segment (start 102.7 73.85) (end 102.7 69) (width 1) (layer "B.Cu") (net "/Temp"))
 (segment (start 118.4 72.55) (end 121.85 72.55) (width 1) (layer "B.Cu") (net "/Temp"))
 (segment (start 105.2 76.35) (end 102.7 73.85) (width 1) (layer "B.Cu") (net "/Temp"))
 (segment (start 111.9 79.5) (end 108.75 76.35) (width 1) (layer "B.Cu") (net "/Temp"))
 (segment (start 118.3 72.45) (end 118.4 72.55) (width 0.2) (layer "B.Cu") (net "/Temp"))
 (segment (start 123.25 73.95) (end 123.25 87.15) (width 1) (layer "B.Cu") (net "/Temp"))
 (segment (start 121.55 88.85) (end 120.29 88.85) (width 1) (layer "B.Cu") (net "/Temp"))
 (segment (start 108.75 76.35) (end 105.2 76.35) (width 1) (layer "B.Cu") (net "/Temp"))
 (segment (start 147.64 78.36) (end 142.27 83.73) (width 1) (layer "B.Cu") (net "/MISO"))
 (segment (start 152.35 78.36) (end 147.64 78.36) (width 1) (layer "B.Cu") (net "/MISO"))
 (segment (start 142.27 83.73) (end 135.55 83.73) (width 1) (layer "B.Cu") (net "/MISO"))
 (segment (start 148 80.9) (end 152.35 80.9) (width 1) (layer "B.Cu") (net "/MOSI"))
 (segment (start 142.63 86.27) (end 148 80.9) (width 1) (layer "B.Cu") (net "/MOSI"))
 (segment (start 135.55 86.27) (end 142.63 86.27) (width 1) (layer "B.Cu") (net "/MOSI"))
 (segment (start 152.35 83.44) (end 147.71 83.44) (width 1) (layer "B.Cu") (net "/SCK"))
 (segment (start 135.69 88.95) (end 135.55 88.81) (width 0.2) (layer "B.Cu") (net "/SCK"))
 (segment (start 145.35 88.2) (end 144.6 88.95) (width 1) (layer "B.Cu") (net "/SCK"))
 (segment (start 144.6 88.95) (end 135.69 88.95) (width 1) (layer "B.Cu") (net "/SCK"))
 (segment (start 147.71 83.44) (end 145.35 85.8) (width 1) (layer "B.Cu") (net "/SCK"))
 (segment (start 145.35 85.8) (end 145.35 88.2) (width 1) (layer "B.Cu") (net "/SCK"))
 (segment (start 149.67 85.98) (end 146.25 89.4) (width 1) (layer "B.Cu") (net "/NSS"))
 (segment (start 120.25 101.4) (end 120.5 101.65) (width 1) (layer "B.Cu") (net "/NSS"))
 (segment (start 146.25 99.5) (end 144.1 101.65) (width 1) (layer "B.Cu") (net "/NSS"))
 (segment (start 120.25 98.97) (end 120.25 101.4) (width 1) (layer "B.Cu") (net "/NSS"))
 (segment (start 144.1 101.65) (end 143.3 101.65) (width 1) (layer "B.Cu") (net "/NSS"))
 (segment (start 146.25 89.4) (end 146.25 99.5) (width 1) (layer "B.Cu") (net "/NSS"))
 (segment (start 152.35 85.98) (end 149.67 85.98) (width 1) (layer "B.Cu") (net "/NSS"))
 (segment (start 120.5 101.65) (end 143.3 101.65) (width 1) (layer "B.Cu") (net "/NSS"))
 (segment (start 118.32 83.73) (end 117.2 84.85) (width 1) (layer "B.Cu") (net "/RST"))
 (segment (start 117.2 84.85) (end 117.2 102.85) (width 1) (layer "B.Cu") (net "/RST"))
 (segment (start 117.2 102.85) (end 118.3 103.95) (width 1) (layer "B.Cu") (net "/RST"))
 (segment (start 120.25 83.73) (end 118.32 83.73) (width 1) (layer "B.Cu") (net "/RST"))
 (segment (start 148.4 102.9) (end 147.35 103.95) (width 1) (layer "B.Cu") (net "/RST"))
 (segment (start 148.4 90.55) (end 148.4 102.9) (width 1) (layer "B.Cu") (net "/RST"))
 (segment (start 150.43 88.52) (end 148.4 90.55) (width 1) (layer "B.Cu") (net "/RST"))
 (segment (start 152.35 88.52) (end 150.43 88.52) (width 1) (layer "B.Cu") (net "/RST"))
 (segment (start 118.3 103.95) (end 143.05 103.95) (width 1) (layer "B.Cu") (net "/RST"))
 (segment (start 147.35 103.95) (end 143.05 103.95) (width 1) (layer "B.Cu") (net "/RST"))
 (segment (start 142.5 63.95) (end 187.9 63.95) (width 1) (layer "B.Cu") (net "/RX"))
 (segment (start 175.062471 112.687529) (end 192.6 95.15) (width 1) (layer "B.Cu") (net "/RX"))
 (segment (start 187.9 63.95) (end 192.6 68.65) (width 1) (layer "B.Cu") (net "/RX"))
 (segment (start 192.6 95.15) (end 192.6 94.6) (width 0.2) (layer "B.Cu") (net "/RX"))
 (segment (start 192.6 68.65) (end 192.6 94.6) (width 1) (layer "B.Cu") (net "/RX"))
 (segment (start 157.591702 112.687529) (end 175.062471 112.687529) (width 1) (layer "B.Cu") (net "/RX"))
 (segment (start 127.1 91.35) (end 128.7 89.75) (width 1) (layer "B.Cu") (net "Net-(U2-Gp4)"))
 (segment (start 120.25 91.35) (end 127.1 91.35) (width 1) (layer "B.Cu") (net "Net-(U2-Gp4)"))
 (segment (start 128.7 89.75) (end 128.7 66.75) (width 1) (layer "B.Cu") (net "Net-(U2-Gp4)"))
 (segment (start 128.7 66.75) (end 131.5 63.95) (width 1) (layer "B.Cu") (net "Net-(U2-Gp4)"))
 (segment (start 182.2 68.45) (end 185.35 68.45) (width 1) (layer "B.Cu") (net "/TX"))
 (segment (start 190.65 92.95) (end 185.2 98.4) (width 1) (layer "B.Cu") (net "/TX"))
 (segment (start 142.1 68.45) (end 182.2 68.45) (width 1) (layer "B.Cu") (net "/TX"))
 (segment (start 185.2 98.4) (end 185.1 98.4) (width 0.2) (layer "B.Cu") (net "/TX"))
 (segment (start 173.352471 110.147529) (end 157.591702 110.147529) (width 1) (layer "B.Cu") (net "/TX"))
 (segment (start 185.35 68.45) (end 190.65 73.75) (width 1) (layer "B.Cu") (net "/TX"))
 (segment (start 185.1 98.4) (end 173.352471 110.147529) (width 1) (layer "B.Cu") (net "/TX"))
 (segment (start 190.65 73.75) (end 190.65 92.95) (width 1) (layer "B.Cu") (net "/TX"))
 (segment (start 131.1 91.35) (end 131.1 68.45) (width 1) (layer "B.Cu") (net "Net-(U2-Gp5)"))
 (segment (start 120.25 93.89) (end 128.56 93.89) (width 1) (layer "B.Cu") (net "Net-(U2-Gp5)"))
 (segment (start 128.56 93.89) (end 131.1 91.35) (width 1) (layer "B.Cu") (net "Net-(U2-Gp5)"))
 (segment (start 171.51 80.94) (end 165.05 87.4) (width 1) (layer "B.Cu") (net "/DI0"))
 (segment (start 165.05 87.4) (end 165.05 95.45) (width 1) (layer "B.Cu") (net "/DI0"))
 (segment (start 114.75 83.1) (end 116.66 81.19) (width 1) (layer "B.Cu") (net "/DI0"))
 (segment (start 154.95 97.3) (end 151.1 101.15) (width 1) (layer "B.Cu") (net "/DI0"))
 (segment (start 148.75 106.7) (end 117.4 106.7) (width 1) (layer "B.Cu") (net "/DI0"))
 (segment (start 114.75 104.05) (end 114.75 83.1) (width 1) (layer "B.Cu") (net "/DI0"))
 (segment (start 178.35 80.94) (end 171.51 80.94) (width 1) (layer "B.Cu") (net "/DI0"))
 (segment (start 117.4 106.7) (end 114.75 104.05) (width 1) (layer "B.Cu") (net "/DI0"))
 (segment (start 165.05 95.45) (end 163.2 97.3) (width 1) (layer "B.Cu") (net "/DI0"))
 (segment (start 151.1 104.35) (end 148.75 106.7) (width 1) (layer "B.Cu") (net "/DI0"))
 (segment (start 151.1 101.15) (end 151.1 104.35) (width 1) (layer "B.Cu") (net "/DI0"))
 (segment (start 163.2 97.3) (end 154.95 97.3) (width 1) (layer "B.Cu") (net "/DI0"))
 (segment (start 116.66 81.19) (end 120.25 81.19) (width 1) (layer "B.Cu") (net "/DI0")))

